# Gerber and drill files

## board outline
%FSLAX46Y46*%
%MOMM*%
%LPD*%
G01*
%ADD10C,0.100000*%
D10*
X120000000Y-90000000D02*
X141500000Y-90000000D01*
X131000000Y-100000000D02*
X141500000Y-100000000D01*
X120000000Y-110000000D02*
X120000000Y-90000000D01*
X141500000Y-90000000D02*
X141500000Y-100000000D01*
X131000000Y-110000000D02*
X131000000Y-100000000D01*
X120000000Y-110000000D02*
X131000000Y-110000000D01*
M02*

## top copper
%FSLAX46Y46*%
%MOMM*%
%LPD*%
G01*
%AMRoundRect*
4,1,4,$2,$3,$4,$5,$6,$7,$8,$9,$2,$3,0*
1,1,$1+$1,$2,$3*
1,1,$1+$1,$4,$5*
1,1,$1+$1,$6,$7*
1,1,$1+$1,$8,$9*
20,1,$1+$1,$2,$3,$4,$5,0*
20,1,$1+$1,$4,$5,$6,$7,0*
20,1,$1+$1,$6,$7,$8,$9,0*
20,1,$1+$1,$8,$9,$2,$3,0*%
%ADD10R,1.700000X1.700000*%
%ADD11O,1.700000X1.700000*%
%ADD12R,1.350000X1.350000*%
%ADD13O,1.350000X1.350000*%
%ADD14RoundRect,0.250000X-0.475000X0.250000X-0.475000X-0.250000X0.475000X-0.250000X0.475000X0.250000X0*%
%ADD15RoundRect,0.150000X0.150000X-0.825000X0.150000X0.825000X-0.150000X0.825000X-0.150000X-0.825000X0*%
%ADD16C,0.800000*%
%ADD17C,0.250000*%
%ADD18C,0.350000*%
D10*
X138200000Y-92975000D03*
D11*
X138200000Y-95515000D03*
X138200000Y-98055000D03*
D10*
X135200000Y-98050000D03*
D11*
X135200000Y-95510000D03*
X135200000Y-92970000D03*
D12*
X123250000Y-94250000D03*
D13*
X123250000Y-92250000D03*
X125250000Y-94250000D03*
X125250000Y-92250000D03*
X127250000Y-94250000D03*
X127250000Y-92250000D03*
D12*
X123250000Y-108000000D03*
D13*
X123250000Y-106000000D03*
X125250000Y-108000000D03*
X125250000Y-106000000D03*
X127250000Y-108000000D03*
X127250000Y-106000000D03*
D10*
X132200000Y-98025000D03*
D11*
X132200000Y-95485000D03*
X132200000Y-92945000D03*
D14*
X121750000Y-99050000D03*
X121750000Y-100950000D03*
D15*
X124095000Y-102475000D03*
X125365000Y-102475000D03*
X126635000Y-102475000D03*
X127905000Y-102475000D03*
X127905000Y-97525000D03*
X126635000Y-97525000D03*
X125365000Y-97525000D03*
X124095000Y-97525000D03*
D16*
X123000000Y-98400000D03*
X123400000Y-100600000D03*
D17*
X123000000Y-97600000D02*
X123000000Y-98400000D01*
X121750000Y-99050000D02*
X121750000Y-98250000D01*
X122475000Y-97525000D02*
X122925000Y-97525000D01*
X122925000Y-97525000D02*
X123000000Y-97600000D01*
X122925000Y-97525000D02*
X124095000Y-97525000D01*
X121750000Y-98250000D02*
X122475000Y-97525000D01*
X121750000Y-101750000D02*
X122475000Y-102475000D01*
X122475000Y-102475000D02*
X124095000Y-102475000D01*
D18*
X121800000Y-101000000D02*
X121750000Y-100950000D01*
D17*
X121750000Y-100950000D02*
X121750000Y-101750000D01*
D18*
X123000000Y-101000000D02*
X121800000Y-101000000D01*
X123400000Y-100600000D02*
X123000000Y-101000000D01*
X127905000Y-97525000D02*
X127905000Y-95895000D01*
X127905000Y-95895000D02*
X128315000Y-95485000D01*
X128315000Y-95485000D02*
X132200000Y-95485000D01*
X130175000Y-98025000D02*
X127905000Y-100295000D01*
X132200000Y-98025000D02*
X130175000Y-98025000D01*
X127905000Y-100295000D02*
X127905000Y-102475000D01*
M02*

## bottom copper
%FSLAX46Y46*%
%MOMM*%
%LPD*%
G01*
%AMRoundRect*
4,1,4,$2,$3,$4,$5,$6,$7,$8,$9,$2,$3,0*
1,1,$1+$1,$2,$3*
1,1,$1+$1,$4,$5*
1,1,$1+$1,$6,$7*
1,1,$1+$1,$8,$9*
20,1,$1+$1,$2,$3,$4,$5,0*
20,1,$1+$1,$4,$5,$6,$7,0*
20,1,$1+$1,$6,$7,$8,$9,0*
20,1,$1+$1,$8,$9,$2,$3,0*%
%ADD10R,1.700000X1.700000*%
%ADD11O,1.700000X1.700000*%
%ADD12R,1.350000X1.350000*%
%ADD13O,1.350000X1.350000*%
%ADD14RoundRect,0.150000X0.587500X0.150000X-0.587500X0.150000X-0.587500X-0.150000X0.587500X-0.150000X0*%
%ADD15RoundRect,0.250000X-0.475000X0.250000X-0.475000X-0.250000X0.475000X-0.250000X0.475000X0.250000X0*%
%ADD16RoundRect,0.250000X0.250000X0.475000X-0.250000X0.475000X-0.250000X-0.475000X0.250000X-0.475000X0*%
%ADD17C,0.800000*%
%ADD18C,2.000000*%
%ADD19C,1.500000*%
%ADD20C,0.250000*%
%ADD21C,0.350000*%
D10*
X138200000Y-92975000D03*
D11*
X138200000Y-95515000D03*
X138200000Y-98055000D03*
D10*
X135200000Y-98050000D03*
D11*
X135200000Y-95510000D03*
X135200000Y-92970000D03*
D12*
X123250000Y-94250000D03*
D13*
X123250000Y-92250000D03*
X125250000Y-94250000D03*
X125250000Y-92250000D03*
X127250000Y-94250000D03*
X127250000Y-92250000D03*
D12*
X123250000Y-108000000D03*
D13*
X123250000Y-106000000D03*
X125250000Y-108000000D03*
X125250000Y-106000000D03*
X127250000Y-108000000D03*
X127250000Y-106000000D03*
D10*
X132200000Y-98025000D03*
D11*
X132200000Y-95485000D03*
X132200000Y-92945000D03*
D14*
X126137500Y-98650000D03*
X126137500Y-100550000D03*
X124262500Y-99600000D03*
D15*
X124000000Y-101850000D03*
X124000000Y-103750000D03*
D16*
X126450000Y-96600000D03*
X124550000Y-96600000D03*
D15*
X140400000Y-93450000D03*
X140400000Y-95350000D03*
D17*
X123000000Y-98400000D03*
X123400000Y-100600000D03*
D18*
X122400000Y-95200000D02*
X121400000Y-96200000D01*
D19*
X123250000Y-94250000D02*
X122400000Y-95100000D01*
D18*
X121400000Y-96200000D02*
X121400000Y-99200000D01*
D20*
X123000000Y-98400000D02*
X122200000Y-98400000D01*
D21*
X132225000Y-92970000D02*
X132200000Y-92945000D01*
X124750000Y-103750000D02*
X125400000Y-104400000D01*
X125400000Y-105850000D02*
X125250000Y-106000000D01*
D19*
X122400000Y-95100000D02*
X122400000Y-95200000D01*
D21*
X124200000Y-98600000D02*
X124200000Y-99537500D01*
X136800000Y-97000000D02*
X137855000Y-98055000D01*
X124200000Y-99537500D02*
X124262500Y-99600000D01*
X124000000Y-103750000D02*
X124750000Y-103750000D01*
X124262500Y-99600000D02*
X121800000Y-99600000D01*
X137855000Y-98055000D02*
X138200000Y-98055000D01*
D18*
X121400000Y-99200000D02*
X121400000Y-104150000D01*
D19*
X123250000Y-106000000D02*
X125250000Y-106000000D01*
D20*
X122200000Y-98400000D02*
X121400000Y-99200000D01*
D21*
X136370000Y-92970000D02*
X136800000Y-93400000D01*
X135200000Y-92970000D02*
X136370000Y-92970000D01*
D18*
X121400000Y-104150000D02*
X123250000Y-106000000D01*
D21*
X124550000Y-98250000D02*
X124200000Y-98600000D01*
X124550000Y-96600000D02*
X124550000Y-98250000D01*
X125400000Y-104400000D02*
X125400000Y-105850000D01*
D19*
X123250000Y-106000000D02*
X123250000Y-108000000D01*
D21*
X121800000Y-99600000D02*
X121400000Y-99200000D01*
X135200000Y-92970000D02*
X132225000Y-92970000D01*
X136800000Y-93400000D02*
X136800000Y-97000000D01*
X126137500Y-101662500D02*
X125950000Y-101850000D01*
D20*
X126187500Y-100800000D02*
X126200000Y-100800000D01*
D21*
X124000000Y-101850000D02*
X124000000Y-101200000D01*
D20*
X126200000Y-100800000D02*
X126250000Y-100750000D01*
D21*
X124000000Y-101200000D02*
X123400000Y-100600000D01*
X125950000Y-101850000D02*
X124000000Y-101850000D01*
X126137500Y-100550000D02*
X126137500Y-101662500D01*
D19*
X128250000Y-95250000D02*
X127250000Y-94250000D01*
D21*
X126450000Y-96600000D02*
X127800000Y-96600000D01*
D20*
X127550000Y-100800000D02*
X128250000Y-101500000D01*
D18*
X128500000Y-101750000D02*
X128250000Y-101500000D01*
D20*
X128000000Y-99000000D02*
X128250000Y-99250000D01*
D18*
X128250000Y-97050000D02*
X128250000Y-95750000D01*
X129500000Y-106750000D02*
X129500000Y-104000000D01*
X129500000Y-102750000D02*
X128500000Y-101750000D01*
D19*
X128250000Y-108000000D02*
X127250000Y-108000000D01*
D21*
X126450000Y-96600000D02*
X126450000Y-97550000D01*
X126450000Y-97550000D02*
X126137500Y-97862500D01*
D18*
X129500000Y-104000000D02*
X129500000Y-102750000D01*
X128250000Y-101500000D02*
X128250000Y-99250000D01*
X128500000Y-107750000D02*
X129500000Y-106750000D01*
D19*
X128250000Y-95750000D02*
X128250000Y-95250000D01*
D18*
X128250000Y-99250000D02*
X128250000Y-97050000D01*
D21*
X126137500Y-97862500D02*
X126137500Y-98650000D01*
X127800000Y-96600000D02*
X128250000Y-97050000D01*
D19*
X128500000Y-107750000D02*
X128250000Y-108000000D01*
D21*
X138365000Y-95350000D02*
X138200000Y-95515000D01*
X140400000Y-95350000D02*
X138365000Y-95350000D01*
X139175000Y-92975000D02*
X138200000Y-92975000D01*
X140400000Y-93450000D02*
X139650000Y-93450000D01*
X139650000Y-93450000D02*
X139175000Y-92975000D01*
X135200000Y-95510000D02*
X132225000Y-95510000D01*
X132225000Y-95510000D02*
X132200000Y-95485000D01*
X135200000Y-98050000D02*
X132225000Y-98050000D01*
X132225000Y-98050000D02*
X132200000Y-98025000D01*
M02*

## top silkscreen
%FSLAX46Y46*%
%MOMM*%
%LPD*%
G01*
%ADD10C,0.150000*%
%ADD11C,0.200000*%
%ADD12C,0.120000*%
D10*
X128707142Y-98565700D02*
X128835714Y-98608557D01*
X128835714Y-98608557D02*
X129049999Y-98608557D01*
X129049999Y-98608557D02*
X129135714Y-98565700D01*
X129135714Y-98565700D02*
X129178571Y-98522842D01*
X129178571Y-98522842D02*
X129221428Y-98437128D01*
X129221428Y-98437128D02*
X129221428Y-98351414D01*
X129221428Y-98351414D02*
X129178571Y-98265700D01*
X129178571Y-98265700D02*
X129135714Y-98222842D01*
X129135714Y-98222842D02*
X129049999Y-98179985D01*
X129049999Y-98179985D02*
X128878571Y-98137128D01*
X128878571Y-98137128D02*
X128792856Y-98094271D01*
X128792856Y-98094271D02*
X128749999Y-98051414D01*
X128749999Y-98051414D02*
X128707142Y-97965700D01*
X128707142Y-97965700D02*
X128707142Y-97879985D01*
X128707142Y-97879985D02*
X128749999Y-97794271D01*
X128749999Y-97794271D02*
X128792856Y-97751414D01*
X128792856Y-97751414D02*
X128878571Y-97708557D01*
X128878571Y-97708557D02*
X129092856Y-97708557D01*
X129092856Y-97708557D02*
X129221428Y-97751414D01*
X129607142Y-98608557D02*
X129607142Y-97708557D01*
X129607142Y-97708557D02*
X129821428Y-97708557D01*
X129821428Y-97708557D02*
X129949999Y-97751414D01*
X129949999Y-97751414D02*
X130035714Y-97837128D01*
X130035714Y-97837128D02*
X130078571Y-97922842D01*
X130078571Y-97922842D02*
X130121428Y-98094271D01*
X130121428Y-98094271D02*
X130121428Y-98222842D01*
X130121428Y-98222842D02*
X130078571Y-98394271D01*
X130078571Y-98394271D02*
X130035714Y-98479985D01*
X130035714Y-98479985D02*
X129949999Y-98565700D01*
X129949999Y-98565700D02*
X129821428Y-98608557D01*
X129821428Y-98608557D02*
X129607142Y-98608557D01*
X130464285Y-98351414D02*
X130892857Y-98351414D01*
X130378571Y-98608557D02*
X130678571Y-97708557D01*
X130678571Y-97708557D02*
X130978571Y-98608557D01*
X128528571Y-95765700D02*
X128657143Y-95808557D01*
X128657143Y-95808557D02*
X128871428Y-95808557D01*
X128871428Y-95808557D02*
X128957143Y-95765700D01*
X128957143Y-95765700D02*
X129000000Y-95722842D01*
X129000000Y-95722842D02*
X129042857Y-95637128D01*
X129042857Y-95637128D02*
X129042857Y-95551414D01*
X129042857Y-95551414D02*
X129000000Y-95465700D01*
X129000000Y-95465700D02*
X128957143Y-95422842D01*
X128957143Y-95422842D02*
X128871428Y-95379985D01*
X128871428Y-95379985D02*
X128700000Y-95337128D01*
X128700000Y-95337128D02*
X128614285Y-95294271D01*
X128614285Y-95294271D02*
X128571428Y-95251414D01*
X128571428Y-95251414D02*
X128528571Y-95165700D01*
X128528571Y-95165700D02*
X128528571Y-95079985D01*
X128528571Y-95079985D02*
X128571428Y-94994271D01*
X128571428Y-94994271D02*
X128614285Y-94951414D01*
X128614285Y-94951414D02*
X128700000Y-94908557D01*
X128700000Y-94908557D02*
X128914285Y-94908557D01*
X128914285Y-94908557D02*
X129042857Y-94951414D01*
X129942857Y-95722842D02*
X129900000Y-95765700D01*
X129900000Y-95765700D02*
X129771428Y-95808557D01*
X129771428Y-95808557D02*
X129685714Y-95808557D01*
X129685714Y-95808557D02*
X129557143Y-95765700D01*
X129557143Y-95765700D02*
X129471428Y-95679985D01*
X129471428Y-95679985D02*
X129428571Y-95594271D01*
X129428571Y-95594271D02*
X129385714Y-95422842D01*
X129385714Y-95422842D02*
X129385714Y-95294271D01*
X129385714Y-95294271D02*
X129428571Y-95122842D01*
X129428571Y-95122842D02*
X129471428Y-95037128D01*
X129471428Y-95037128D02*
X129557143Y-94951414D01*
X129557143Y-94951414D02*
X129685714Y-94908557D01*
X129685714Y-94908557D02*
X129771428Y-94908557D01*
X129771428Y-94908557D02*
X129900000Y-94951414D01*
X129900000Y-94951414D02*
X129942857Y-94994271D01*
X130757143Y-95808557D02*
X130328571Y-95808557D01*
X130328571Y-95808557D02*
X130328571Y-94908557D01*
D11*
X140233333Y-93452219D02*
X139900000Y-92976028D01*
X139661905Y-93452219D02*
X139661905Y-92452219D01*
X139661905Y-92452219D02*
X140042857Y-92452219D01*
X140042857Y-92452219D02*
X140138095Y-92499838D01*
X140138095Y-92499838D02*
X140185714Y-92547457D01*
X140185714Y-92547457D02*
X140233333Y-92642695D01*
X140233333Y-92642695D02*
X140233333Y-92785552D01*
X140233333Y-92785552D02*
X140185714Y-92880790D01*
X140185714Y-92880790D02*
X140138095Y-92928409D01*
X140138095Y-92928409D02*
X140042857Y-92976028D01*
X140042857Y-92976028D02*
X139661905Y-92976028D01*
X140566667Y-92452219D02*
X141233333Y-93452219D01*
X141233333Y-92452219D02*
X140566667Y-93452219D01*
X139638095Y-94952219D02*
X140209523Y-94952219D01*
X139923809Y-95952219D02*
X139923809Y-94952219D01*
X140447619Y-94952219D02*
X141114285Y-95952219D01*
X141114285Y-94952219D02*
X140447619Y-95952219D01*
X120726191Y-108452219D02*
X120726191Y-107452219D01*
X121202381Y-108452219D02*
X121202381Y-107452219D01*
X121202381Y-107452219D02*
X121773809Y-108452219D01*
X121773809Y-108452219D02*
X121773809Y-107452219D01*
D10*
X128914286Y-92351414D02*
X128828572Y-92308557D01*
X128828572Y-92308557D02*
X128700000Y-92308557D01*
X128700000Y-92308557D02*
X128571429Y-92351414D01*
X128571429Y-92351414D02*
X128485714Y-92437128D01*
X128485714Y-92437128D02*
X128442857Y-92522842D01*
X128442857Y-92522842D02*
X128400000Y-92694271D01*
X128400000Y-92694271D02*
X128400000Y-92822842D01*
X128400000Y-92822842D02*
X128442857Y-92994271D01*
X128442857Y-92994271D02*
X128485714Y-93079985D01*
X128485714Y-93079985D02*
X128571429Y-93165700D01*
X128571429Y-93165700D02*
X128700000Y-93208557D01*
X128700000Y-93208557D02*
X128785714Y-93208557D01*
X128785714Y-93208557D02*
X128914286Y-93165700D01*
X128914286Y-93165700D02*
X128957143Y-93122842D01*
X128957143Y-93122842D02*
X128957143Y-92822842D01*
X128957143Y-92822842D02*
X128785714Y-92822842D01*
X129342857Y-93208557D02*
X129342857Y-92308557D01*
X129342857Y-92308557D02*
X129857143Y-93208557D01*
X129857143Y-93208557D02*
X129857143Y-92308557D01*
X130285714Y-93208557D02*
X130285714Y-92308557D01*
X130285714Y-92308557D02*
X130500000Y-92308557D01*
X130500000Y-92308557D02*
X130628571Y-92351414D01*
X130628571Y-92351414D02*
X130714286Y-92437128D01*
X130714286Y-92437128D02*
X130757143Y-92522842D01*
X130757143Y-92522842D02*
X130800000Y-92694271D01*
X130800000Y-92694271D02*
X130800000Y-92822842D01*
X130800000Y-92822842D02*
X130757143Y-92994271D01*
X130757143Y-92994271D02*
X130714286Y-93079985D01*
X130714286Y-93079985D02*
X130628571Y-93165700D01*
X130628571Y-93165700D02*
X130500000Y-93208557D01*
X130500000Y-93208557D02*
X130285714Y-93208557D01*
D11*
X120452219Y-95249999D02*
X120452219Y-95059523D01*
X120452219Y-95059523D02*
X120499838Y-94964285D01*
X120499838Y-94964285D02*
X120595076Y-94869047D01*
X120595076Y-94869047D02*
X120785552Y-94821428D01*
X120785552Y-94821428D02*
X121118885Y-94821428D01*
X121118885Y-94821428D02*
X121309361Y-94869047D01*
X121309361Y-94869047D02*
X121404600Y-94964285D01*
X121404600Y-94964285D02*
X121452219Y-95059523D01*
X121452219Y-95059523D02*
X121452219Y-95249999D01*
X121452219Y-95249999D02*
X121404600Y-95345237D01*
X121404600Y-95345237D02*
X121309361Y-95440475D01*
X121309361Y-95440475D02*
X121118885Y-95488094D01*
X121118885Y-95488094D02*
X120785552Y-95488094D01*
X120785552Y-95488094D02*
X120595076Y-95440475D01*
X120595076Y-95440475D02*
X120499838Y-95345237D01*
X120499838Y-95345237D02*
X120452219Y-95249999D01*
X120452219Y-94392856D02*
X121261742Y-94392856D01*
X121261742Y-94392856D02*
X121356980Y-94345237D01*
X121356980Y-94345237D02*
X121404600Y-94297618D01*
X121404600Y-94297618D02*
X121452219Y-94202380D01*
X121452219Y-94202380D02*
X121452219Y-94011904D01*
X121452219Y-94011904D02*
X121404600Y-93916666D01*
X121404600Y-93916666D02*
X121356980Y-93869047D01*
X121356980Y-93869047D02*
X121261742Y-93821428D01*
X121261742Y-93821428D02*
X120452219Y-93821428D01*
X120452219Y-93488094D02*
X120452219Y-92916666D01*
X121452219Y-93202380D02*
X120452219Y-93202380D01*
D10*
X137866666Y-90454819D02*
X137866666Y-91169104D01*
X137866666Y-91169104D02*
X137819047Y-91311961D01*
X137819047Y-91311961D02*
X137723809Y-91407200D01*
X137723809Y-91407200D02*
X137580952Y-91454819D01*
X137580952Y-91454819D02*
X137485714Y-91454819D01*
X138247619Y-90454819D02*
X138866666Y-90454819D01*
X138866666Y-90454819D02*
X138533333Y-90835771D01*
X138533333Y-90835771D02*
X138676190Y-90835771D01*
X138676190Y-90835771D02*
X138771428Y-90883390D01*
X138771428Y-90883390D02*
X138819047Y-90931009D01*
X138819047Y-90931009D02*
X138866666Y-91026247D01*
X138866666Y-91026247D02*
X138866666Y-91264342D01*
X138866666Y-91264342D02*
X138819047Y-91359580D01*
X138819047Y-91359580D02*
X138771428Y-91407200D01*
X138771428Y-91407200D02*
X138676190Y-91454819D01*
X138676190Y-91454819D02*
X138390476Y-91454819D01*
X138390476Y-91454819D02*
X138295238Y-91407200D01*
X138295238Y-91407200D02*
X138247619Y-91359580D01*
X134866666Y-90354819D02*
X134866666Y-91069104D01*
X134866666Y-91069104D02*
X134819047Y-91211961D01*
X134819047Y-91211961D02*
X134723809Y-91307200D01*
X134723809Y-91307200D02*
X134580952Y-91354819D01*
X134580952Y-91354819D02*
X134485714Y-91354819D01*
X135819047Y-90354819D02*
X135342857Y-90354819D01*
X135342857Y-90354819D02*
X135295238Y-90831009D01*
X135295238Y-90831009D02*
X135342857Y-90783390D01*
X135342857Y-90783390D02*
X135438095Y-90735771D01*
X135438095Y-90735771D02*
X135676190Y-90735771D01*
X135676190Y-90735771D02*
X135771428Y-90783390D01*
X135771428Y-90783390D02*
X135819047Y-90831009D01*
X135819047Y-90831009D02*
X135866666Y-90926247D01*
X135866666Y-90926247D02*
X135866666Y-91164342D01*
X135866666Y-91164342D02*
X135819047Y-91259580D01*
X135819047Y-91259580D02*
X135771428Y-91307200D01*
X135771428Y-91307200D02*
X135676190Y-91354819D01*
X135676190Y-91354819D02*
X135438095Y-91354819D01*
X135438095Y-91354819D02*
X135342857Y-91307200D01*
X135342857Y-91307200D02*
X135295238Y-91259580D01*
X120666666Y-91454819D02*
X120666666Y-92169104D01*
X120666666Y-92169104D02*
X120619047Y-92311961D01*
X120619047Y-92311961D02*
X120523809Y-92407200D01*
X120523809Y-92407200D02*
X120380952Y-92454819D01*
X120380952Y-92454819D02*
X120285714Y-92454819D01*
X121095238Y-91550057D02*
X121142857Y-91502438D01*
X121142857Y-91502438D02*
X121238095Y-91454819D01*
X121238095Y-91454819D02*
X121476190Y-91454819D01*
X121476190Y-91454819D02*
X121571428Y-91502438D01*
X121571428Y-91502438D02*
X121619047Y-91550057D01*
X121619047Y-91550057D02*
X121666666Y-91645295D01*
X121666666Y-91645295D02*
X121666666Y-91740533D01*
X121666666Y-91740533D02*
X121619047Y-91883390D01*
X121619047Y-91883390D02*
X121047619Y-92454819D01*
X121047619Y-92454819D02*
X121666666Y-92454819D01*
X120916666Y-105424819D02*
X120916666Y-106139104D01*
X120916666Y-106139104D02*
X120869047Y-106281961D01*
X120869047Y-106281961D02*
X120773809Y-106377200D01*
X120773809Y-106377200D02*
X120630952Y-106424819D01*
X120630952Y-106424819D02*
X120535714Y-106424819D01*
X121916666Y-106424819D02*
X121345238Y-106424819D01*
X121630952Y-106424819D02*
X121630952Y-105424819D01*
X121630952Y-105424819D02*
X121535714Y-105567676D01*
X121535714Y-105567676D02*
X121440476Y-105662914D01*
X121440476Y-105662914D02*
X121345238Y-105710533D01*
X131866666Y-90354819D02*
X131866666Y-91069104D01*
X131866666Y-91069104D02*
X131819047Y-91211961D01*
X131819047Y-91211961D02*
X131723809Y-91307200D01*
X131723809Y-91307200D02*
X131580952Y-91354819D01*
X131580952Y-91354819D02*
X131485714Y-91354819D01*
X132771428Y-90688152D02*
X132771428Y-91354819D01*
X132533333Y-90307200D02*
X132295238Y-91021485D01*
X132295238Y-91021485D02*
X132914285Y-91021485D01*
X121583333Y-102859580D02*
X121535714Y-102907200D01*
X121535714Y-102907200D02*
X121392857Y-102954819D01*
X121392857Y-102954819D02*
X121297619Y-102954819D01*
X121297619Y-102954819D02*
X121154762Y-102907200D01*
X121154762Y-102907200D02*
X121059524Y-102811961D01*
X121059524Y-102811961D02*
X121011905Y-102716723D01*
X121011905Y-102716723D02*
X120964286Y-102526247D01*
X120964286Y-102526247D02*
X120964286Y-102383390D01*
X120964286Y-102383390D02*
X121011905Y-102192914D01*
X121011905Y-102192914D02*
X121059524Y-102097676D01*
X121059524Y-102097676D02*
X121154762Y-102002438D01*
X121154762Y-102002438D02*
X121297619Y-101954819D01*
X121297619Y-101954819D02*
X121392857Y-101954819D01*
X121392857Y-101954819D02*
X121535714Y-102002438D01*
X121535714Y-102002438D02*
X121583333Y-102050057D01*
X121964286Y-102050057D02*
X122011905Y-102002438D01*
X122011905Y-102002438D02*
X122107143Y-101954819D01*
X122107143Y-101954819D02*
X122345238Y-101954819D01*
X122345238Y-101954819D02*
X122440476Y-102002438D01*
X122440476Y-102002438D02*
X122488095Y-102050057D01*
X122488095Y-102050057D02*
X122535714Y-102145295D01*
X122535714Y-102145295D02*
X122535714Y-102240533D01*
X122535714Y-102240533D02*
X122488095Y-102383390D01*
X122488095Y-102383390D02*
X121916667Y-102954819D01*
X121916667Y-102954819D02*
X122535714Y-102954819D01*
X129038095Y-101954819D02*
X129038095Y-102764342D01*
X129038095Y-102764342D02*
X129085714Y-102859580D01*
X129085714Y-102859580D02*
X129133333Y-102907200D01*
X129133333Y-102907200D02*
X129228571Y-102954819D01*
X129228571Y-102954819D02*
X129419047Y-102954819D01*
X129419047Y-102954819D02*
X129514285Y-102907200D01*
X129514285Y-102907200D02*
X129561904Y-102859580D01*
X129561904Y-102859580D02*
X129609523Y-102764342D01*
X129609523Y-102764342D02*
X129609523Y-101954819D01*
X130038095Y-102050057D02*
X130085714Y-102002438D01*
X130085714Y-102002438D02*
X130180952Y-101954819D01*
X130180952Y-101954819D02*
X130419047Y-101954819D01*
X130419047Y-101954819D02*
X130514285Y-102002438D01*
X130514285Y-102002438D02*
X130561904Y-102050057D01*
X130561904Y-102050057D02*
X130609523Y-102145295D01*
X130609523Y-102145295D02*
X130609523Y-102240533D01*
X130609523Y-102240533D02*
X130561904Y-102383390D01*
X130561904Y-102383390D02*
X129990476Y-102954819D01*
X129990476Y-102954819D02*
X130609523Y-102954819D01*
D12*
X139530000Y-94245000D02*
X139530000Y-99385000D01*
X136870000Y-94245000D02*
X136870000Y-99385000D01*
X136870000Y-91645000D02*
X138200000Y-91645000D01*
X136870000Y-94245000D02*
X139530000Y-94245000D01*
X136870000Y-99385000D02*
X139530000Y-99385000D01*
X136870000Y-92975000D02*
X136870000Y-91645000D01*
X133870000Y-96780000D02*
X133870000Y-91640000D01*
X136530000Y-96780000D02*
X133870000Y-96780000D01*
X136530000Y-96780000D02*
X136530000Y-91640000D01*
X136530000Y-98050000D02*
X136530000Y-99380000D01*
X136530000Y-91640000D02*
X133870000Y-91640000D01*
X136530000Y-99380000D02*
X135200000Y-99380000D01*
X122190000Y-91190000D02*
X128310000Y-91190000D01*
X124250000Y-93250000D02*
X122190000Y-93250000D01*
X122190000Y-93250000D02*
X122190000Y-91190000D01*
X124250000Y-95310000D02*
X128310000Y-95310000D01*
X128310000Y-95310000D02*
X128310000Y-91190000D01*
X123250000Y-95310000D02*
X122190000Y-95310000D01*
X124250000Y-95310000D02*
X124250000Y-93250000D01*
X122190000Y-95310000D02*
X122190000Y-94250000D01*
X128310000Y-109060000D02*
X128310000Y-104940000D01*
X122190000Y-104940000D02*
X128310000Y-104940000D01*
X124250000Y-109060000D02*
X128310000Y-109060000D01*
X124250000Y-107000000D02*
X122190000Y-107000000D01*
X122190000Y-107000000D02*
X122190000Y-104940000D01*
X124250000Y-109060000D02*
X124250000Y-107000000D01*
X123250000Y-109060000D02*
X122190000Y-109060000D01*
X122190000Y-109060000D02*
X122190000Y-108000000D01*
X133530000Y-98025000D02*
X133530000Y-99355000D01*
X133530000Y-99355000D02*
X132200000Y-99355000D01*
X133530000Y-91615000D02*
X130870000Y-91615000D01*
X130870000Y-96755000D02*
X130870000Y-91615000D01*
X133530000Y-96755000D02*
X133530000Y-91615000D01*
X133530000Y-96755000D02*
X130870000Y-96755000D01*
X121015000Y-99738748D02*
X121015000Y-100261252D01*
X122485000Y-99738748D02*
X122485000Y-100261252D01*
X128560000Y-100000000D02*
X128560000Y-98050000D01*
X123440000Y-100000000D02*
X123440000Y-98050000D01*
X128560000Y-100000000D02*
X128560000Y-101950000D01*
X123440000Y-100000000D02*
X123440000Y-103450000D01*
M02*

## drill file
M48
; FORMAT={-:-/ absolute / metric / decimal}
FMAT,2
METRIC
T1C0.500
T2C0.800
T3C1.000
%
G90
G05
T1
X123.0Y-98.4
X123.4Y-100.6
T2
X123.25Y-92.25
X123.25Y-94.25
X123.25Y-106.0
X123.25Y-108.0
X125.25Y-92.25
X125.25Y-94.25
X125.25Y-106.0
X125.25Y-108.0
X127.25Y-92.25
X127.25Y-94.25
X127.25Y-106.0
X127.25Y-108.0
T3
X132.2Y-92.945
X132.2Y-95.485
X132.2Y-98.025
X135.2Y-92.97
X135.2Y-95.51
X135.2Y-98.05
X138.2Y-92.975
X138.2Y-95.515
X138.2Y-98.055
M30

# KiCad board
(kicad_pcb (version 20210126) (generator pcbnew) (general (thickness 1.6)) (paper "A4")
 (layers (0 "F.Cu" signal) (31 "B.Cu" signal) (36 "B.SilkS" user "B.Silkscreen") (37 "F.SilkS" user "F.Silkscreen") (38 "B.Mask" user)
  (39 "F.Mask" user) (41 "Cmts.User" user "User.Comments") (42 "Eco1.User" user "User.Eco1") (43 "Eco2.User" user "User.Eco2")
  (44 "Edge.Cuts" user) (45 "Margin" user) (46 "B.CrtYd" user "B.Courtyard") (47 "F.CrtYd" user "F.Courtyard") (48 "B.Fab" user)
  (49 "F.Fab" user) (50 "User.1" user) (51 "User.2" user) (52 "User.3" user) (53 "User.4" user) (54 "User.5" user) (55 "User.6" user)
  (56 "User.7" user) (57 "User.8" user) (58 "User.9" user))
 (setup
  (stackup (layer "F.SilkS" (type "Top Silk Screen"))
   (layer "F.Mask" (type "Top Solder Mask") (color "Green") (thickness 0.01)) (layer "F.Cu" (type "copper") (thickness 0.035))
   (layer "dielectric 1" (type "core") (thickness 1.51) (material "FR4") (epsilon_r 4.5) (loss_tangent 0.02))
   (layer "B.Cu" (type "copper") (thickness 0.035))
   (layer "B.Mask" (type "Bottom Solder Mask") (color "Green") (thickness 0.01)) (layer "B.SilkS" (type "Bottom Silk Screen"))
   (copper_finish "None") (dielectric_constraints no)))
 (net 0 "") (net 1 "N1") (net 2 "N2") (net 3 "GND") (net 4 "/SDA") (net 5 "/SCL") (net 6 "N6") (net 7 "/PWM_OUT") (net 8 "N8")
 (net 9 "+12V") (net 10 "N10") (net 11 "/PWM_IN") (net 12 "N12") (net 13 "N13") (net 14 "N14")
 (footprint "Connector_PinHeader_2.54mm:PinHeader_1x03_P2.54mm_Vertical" (layer "F.Cu") (at 138.2 92.975)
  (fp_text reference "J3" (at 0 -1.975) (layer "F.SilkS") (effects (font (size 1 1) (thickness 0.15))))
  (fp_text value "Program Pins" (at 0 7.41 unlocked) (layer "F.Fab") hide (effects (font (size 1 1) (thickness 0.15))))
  (fp_line (start 1.33 1.27) (end 1.33 6.41) (layer "F.SilkS") (width 0.12))
  (fp_line (start -1.33 1.27) (end -1.33 6.41) (layer "F.SilkS") (width 0.12))
  (fp_line (start -1.33 -1.33) (end 0 -1.33) (layer "F.SilkS") (width 0.12))
  (fp_line (start -1.33 1.27) (end 1.33 1.27) (layer "F.SilkS") (width 0.12))
  (fp_line (start -1.33 6.41) (end 1.33 6.41) (layer "F.SilkS") (width 0.12))
  (fp_line (start -1.33 0) (end -1.33 -1.33) (layer "F.SilkS") (width 0.12))
  (pad "1" thru_hole rect (at 0 0) (locked) (size 1.7 1.7) (drill 1) (layers *.Cu *.Mask) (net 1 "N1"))
  (pad "2" thru_hole oval (at 0 2.54) (locked) (size 1.7 1.7) (drill 1) (layers *.Cu *.Mask) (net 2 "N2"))
  (pad "3" thru_hole oval (at 0 5.08) (locked) (size 1.7 1.7) (drill 1) (layers *.Cu *.Mask) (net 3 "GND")))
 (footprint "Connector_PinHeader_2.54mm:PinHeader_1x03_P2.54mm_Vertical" (layer "F.Cu") (at 135.2 98.05 180)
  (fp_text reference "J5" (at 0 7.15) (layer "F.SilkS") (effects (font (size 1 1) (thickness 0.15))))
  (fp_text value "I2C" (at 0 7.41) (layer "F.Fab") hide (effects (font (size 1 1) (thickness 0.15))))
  (fp_line (start 1.33 1.27) (end 1.33 6.41) (layer "F.SilkS") (width 0.12))
  (fp_line (start -1.33 1.27) (end 1.33 1.27) (layer "F.SilkS") (width 0.12))
  (fp_line (start -1.33 1.27) (end -1.33 6.41) (layer "F.SilkS") (width 0.12))
  (fp_line (start -1.33 0) (end -1.33 -1.33) (layer "F.SilkS") (width 0.12))
  (fp_line (start -1.33 6.41) (end 1.33 6.41) (layer "F.SilkS") (width 0.12))
  (fp_line (start -1.33 -1.33) (end 0 -1.33) (layer "F.SilkS") (width 0.12))
  (pad "1" thru_hole rect (at 0 0 180) (locked) (size 1.7 1.7) (drill 1) (layers *.Cu *.Mask) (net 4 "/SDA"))
  (pad "2" thru_hole oval (at 0 2.54 180) (locked) (size 1.7 1.7) (drill 1) (layers *.Cu *.Mask) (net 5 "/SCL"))
  (pad "3" thru_hole oval (at 0 5.08 180) (locked) (size 1.7 1.7) (drill 1) (layers *.Cu *.Mask) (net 3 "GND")))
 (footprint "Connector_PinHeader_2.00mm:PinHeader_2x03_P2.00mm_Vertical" (layer "F.Cu") (at 123.25 94.25 90)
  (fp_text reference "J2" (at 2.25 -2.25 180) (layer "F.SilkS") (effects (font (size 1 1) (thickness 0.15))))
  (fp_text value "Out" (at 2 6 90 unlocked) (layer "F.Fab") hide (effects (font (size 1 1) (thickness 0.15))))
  (fp_line (start 3.06 -1.06) (end 3.06 5.06) (layer "F.SilkS") (width 0.12))
  (fp_line (start 1 1) (end 1 -1.06) (layer "F.SilkS") (width 0.12))
  (fp_line (start 1 -1.06) (end 3.06 -1.06) (layer "F.SilkS") (width 0.12))
  (fp_line (start -1.06 1) (end -1.06 5.06) (layer "F.SilkS") (width 0.12))
  (fp_line (start -1.06 5.06) (end 3.06 5.06) (layer "F.SilkS") (width 0.12))
  (fp_line (start -1.06 0) (end -1.06 -1.06) (layer "F.SilkS") (width 0.12))
  (fp_line (start -1.06 1) (end 1 1) (layer "F.SilkS") (width 0.12))
  (fp_line (start -1.06 -1.06) (end 0 -1.06) (layer "F.SilkS") (width 0.12))
  (pad "1" thru_hole rect (at 0 0 90) (locked) (size 1.35 1.35) (drill 0.8) (layers *.Cu *.Mask) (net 3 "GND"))
  (pad "2" thru_hole oval (at 2 0 90) (locked) (size 1.35 1.35) (drill 0.8) (layers *.Cu *.Mask) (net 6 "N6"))
  (pad "3" thru_hole oval (at 0 2 90) (locked) (size 1.35 1.35) (drill 0.8) (layers *.Cu *.Mask) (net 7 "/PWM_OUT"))
  (pad "4" thru_hole oval (at 2 2 90) (locked) (size 1.35 1.35) (drill 0.8) (layers *.Cu *.Mask) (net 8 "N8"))
  (pad "5" thru_hole oval (at 0 4 90) (locked) (size 1.35 1.35) (drill 0.8) (layers *.Cu *.Mask) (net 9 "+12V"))
  (pad "6" thru_hole oval (at 2 4 90) (locked) (size 1.35 1.35) (drill 0.8) (layers *.Cu *.Mask) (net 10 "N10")))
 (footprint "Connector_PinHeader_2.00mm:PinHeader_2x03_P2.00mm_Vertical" (layer "F.Cu") (at 123.25 108 90)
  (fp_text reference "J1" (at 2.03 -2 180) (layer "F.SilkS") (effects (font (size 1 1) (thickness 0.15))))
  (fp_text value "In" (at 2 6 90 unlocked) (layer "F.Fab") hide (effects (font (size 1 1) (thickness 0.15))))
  (fp_line (start -1.06 5.06) (end 3.06 5.06) (layer "F.SilkS") (width 0.12))
  (fp_line (start 3.06 -1.06) (end 3.06 5.06) (layer "F.SilkS") (width 0.12))
  (fp_line (start -1.06 1) (end -1.06 5.06) (layer "F.SilkS") (width 0.12))
  (fp_line (start 1 1) (end 1 -1.06) (layer "F.SilkS") (width 0.12))
  (fp_line (start 1 -1.06) (end 3.06 -1.06) (layer "F.SilkS") (width 0.12))
  (fp_line (start -1.06 1) (end 1 1) (layer "F.SilkS") (width 0.12))
  (fp_line (start -1.06 0) (end -1.06 -1.06) (layer "F.SilkS") (width 0.12))
  (fp_line (start -1.06 -1.06) (end 0 -1.06) (layer "F.SilkS") (width 0.12))
  (pad "1" thru_hole rect (at 0 0 90) (locked) (size 1.35 1.35) (drill 0.8) (layers *.Cu *.Mask) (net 3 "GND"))
  (pad "2" thru_hole oval (at 2 0 90) (locked) (size 1.35 1.35) (drill 0.8) (layers *.Cu *.Mask) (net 3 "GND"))
  (pad "3" thru_hole oval (at 0 2 90) (locked) (size 1.35 1.35) (drill 0.8) (layers *.Cu *.Mask) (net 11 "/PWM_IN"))
  (pad "4" thru_hole oval (at 2 2 90) (locked) (size 1.35 1.35) (drill 0.8) (layers *.Cu *.Mask) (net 3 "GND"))
  (pad "5" thru_hole oval (at 0 4 90) (locked) (size 1.35 1.35) (drill 0.8) (layers *.Cu *.Mask) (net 9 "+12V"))
  (pad "6" thru_hole oval (at 2 4 90) (locked) (size 1.35 1.35) (drill 0.8) (layers *.Cu *.Mask) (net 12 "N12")))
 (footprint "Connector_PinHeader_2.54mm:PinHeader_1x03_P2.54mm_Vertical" (layer "F.Cu") (at 132.2 98.025 180)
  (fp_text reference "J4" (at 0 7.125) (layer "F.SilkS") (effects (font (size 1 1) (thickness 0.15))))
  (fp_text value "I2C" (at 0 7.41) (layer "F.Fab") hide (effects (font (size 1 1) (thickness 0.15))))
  (fp_line (start -1.33 0) (end -1.33 -1.33) (layer "F.SilkS") (width 0.12))
  (fp_line (start -1.33 -1.33) (end 0 -1.33) (layer "F.SilkS") (width 0.12))
  (fp_line (start -1.33 6.41) (end 1.33 6.41) (layer "F.SilkS") (width 0.12))
  (fp_line (start 1.33 1.27) (end 1.33 6.41) (layer "F.SilkS") (width 0.12))
  (fp_line (start -1.33 1.27) (end -1.33 6.41) (layer "F.SilkS") (width 0.12))
  (fp_line (start -1.33 1.27) (end 1.33 1.27) (layer "F.SilkS") (width 0.12))
  (pad "1" thru_hole rect (at 0 0 180) (locked) (size 1.7 1.7) (drill 1) (layers *.Cu *.Mask) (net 4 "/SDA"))
  (pad "2" thru_hole oval (at 0 2.54 180) (locked) (size 1.7 1.7) (drill 1) (layers *.Cu *.Mask) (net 5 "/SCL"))
  (pad "3" thru_hole oval (at 0 5.08 180) (locked) (size 1.7 1.7) (drill 1) (layers *.Cu *.Mask) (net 3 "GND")))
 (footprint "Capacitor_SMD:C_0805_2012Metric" (layer "F.Cu") (at 121.75 100 -90)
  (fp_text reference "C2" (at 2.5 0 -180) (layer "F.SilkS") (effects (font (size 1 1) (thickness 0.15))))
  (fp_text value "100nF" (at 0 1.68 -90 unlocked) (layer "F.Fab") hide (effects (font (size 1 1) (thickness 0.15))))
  (fp_line (start -0.261252 0.735) (end 0.261252 0.735) (layer "F.SilkS") (width 0.12))
  (fp_line (start -0.261252 -0.735) (end 0.261252 -0.735) (layer "F.SilkS") (width 0.12))
  (pad "1" smd roundrect (at -0.95 0 270) (locked) (size 1 1.45) (layers "F.Cu" "F.Paste" "F.Mask") (roundrect_rratio 0.25) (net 3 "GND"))
  (pad "2" smd roundrect (at 0.95 0 270) (locked) (size 1 1.45) (layers "F.Cu" "F.Paste" "F.Mask") (roundrect_rratio 0.25) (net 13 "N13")))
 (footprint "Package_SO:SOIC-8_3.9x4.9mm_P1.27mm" (layer "F.Cu") (at 126 100 90)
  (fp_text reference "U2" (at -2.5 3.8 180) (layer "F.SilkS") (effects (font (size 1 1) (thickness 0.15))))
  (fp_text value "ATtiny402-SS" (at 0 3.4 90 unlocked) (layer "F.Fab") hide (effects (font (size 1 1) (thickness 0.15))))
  (fp_line (start 0 2.56) (end 1.95 2.56) (layer "F.SilkS") (width 0.12))
  (fp_line (start 0 -2.56) (end 1.95 -2.56) (layer "F.SilkS") (width 0.12))
  (fp_line (start 0 2.56) (end -1.95 2.56) (layer "F.SilkS") (width 0.12))
  (fp_line (start 0 -2.56) (end -3.45 -2.56) (layer "F.SilkS") (width 0.12))
  (pad "1" smd roundrect (at -2.475 -1.905 90) (locked) (size 1.95 0.6) (layers "F.Cu" "F.Paste" "F.Mask") (roundrect_rratio 0.25)
   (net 13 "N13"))
  (pad "2" smd roundrect (at -2.475 -0.635 90) (locked) (size 1.95 0.6) (layers "F.Cu" "F.Paste" "F.Mask") (roundrect_rratio 0.25)
   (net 11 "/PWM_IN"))
  (pad "3" smd roundrect (at -2.475 0.635 90) (locked) (size 1.95 0.6) (layers "F.Cu" "F.Paste" "F.Mask") (roundrect_rratio 0.25)
   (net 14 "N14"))
  (pad "4" smd roundrect (at -2.475 1.905 90) (locked) (size 1.95 0.6) (layers "F.Cu" "F.Paste" "F.Mask") (roundrect_rratio 0.25)
   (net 4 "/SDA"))
  (pad "5" smd roundrect (at 2.475 1.905 90) (locked) (size 1.95 0.6) (layers "F.Cu" "F.Paste" "F.Mask") (roundrect_rratio 0.25)
   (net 5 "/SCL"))
  (pad "6" smd roundrect (at 2.475 0.635 90) (locked) (size 1.95 0.6) (layers "F.Cu" "F.Paste" "F.Mask") (roundrect_rratio 0.25)
   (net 2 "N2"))
  (pad "7" smd roundrect (at 2.475 -0.635 90) (locked) (size 1.95 0.6) (layers "F.Cu" "F.Paste" "F.Mask") (roundrect_rratio 0.25)
   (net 7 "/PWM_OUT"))
  (pad "8" smd roundrect (at 2.475 -1.905 90) (locked) (size 1.95 0.6) (layers "F.Cu" "F.Paste" "F.Mask") (roundrect_rratio 0.25)
   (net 3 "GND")))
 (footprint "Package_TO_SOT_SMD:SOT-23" (layer "B.Cu") (at 125.2 99.6 180)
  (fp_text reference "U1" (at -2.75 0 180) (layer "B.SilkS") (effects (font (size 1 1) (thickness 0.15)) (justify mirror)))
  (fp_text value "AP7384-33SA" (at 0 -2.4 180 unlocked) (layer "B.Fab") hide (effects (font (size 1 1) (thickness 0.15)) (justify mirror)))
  (pad "1" smd roundrect (at -0.9375 0.95 180) (locked) (size 1.475 0.6) (layers "B.Cu" "B.Paste" "B.Mask") (roundrect_rratio 0.25)
   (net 9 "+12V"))
  (pad "2" smd roundrect (at -0.9375 -0.95 180) (locked) (size 1.475 0.6) (layers "B.Cu" "B.Paste" "B.Mask") (roundrect_rratio 0.25)
   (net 13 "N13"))
  (pad "3" smd roundrect (at 0.9375 0 180) (locked) (size 1.475 0.6) (layers "B.Cu" "B.Paste" "B.Mask") (roundrect_rratio 0.25)
   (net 3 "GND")))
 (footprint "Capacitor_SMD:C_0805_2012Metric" (layer "B.Cu") (at 124 102.8 -90)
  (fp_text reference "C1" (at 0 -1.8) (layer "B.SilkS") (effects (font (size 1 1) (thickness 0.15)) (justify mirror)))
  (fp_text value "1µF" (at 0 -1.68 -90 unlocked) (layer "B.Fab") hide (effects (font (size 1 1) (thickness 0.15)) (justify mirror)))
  (pad "1" smd roundrect (at -0.95 0 270) (locked) (size 1 1.45) (layers "B.Cu" "B.Paste" "B.Mask") (roundrect_rratio 0.25) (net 13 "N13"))
  (pad "2" smd roundrect (at 0.95 0 270) (locked) (size 1 1.45) (layers "B.Cu" "B.Paste" "B.Mask") (roundrect_rratio 0.25) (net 3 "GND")))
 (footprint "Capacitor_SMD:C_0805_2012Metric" (layer "B.Cu") (at 125.5 96.6 180)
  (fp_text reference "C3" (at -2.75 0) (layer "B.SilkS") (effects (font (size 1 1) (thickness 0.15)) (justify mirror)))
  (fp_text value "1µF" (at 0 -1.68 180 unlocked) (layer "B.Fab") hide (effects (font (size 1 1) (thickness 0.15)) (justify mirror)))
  (pad "1" smd roundrect (at -0.95 0 180) (locked) (size 1 1.45) (layers "B.Cu" "B.Paste" "B.Mask") (roundrect_rratio 0.25) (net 9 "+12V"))
  (pad "2" smd roundrect (at 0.95 0 180) (locked) (size 1 1.45) (layers "B.Cu" "B.Paste" "B.Mask") (roundrect_rratio 0.25) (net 3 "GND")))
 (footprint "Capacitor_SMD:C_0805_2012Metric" (layer "B.Cu") (at 140.4 94.4 -90)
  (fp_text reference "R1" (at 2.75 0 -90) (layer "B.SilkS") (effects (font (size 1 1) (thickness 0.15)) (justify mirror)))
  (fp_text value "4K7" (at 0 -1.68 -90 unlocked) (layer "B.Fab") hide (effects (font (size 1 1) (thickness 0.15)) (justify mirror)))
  (pad "1" smd roundrect (at -0.95 0 270) (locked) (size 1 1.45) (layers "B.Cu" "B.Paste" "B.Mask") (roundrect_rratio 0.25) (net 1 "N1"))
  (pad "2" smd roundrect (at 0.95 0 270) (locked) (size 1 1.45) (layers "B.Cu" "B.Paste" "B.Mask") (roundrect_rratio 0.25) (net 2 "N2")))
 (gr_line (start 120 90) (end 141.5 90) (layer "Edge.Cuts") (width 0.1))
 (gr_line (start 131 100) (end 141.5 100) (layer "Edge.Cuts") (width 0.1))
 (gr_line (start 120 110) (end 120 90) (layer "Edge.Cuts") (width 0.1))
 (gr_line (start 141.5 90) (end 141.5 100) (layer "Edge.Cuts") (width 0.1))
 (gr_line (start 131 110) (end 131 100) (layer "Edge.Cuts") (width 0.1))
 (gr_line (start 120 110) (end 131 110) (layer "Edge.Cuts") (width 0.1))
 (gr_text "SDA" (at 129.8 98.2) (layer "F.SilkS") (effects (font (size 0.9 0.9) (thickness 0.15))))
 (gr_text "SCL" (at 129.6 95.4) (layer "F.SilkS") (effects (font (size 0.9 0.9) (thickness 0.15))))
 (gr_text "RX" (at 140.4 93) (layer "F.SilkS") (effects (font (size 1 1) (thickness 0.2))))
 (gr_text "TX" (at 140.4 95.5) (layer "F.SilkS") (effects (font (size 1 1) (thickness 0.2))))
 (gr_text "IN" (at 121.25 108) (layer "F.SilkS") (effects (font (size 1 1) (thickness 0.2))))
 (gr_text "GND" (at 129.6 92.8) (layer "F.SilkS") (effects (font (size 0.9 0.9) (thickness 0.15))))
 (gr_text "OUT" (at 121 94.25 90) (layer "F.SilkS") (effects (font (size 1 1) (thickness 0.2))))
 (segment (start 123 97.6) (end 123 98.4) (width 0.25) (layer "F.Cu") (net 3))
 (segment (start 121.75 99.05) (end 121.75 98.25) (width 0.25) (layer "F.Cu") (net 3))
 (segment (start 122.475 97.525) (end 122.925 97.525) (width 0.25) (layer "F.Cu") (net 3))
 (segment (start 122.925 97.525) (end 123 97.6) (width 0.25) (layer "F.Cu") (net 3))
 (segment (start 122.925 97.525) (end 124.095 97.525) (width 0.25) (layer "F.Cu") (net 3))
 (segment (start 121.75 98.25) (end 122.475 97.525) (width 0.25) (layer "F.Cu") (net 3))
 (via (at 123 98.4) (size 0.8) (drill 0.5) (layers "F.Cu" "B.Cu") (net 3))
 (segment (start 122.4 95.2) (end 121.4 96.2) (width 2) (layer "B.Cu") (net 3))
 (segment (start 123.25 94.25) (end 122.4 95.1) (width 1.5) (layer "B.Cu") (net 3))
 (segment (start 121.4 96.2) (end 121.4 99.2) (width 2) (layer "B.Cu") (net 3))
 (segment (start 123 98.4) (end 122.2 98.4) (width 0.25) (layer "B.Cu") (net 3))
 (segment (start 132.225 92.97) (end 132.2 92.945) (width 0.35) (layer "B.Cu") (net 3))
 (segment (start 124.75 103.75) (end 125.4 104.4) (width 0.35) (layer "B.Cu") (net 3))
 (segment (start 125.4 105.85) (end 125.25 106) (width 0.35) (layer "B.Cu") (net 3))
 (segment (start 122.4 95.1) (end 122.4 95.2) (width 1.5) (layer "B.Cu") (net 3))
 (segment (start 124.2 98.6) (end 124.2 99.5375) (width 0.35) (layer "B.Cu") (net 3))
 (segment (start 136.8 97) (end 137.855 98.055) (width 0.35) (layer "B.Cu") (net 3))
 (segment (start 124.2 99.5375) (end 124.2625 99.6) (width 0.35) (layer "B.Cu") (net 3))
 (segment (start 124 103.75) (end 124.75 103.75) (width 0.35) (layer "B.Cu") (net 3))
 (segment (start 124.2625 99.6) (end 121.8 99.6) (width 0.35) (layer "B.Cu") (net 3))
 (segment (start 137.855 98.055) (end 138.2 98.055) (width 0.35) (layer "B.Cu") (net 3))
 (segment (start 121.4 99.2) (end 121.4 104.15) (width 2) (layer "B.Cu") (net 3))
 (segment (start 123.25 106) (end 125.25 106) (width 1.5) (layer "B.Cu") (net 3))
 (segment (start 122.2 98.4) (end 121.4 99.2) (width 0.25) (layer "B.Cu") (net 3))
 (segment (start 136.37 92.97) (end 136.8 93.4) (width 0.35) (layer "B.Cu") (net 3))
 (segment (start 135.2 92.97) (end 136.37 92.97) (width 0.35) (layer "B.Cu") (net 3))
 (segment (start 121.4 104.15) (end 123.25 106) (width 2) (layer "B.Cu") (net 3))
 (segment (start 124.55 98.25) (end 124.2 98.6) (width 0.35) (layer "B.Cu") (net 3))
 (segment (start 124.55 96.6) (end 124.55 98.25) (width 0.35) (layer "B.Cu") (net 3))
 (segment (start 125.4 104.4) (end 125.4 105.85) (width 0.35) (layer "B.Cu") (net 3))
 (segment (start 123.25 106) (end 123.25 108) (width 1.5) (layer "B.Cu") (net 3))
 (segment (start 121.8 99.6) (end 121.4 99.2) (width 0.35) (layer "B.Cu") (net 3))
 (segment (start 135.2 92.97) (end 132.225 92.97) (width 0.35) (layer "B.Cu") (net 3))
 (segment (start 136.8 93.4) (end 136.8 97) (width 0.35) (layer "B.Cu") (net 3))
 (segment (start 121.75 101.75) (end 122.475 102.475) (width 0.25) (layer "F.Cu") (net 13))
 (segment (start 122.475 102.475) (end 124.095 102.475) (width 0.25) (layer "F.Cu") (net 13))
 (segment (start 121.8 101) (end 121.75 100.95) (width 0.35) (layer "F.Cu") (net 13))
 (segment (start 121.75 100.95) (end 121.75 101.75) (width 0.25) (layer "F.Cu") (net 13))
 (segment (start 123 101) (end 121.8 101) (width 0.35) (layer "F.Cu") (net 13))
 (segment (start 123.4 100.6) (end 123 101) (width 0.35) (layer "F.Cu") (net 13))
 (via (at 123.4 100.6) (size 0.8) (drill 0.5) (layers "F.Cu" "B.Cu") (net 13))
 (segment (start 126.1375 101.6625) (end 125.95 101.85) (width 0.35) (layer "B.Cu") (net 13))
 (segment (start 126.1875 100.8) (end 126.2 100.8) (width 0.25) (layer "B.Cu") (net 13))
 (segment (start 124 101.85) (end 124 101.2) (width 0.35) (layer "B.Cu") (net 13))
 (segment (start 126.2 100.8) (end 126.25 100.75) (width 0.25) (layer "B.Cu") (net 13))
 (segment (start 124 101.2) (end 123.4 100.6) (width 0.35) (layer "B.Cu") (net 13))
 (segment (start 125.95 101.85) (end 124 101.85) (width 0.35) (layer "B.Cu") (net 13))
 (segment (start 126.1375 100.55) (end 126.1375 101.6625) (width 0.35) (layer "B.Cu") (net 13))
 (segment (start 128.25 95.25) (end 127.25 94.25) (width 1.5) (layer "B.Cu") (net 9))
 (segment (start 126.45 96.6) (end 127.8 96.6) (width 0.35) (layer "B.Cu") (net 9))
 (segment (start 127.55 100.8) (end 128.25 101.5) (width 0.25) (layer "B.Cu") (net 9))
 (segment (start 128.5 101.75) (end 128.25 101.5) (width 2) (layer "B.Cu") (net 9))
 (segment (start 128 99) (end 128.25 99.25) (width 0.25) (layer "B.Cu") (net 9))
 (segment (start 128.25 97.05) (end 128.25 95.75) (width 2) (layer "B.Cu") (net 9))
 (segment (start 129.5 106.75) (end 129.5 104) (width 2) (layer "B.Cu") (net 9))
 (segment (start 129.5 102.75) (end 128.5 101.75) (width 2) (layer "B.Cu") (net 9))
 (segment (start 128.25 108) (end 127.25 108) (width 1.5) (layer "B.Cu") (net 9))
 (segment (start 126.45 96.6) (end 126.45 97.55) (width 0.35) (layer "B.Cu") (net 9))
 (segment (start 126.45 97.55) (end 126.1375 97.8625) (width 0.35) (layer "B.Cu") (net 9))
 (segment (start 129.5 104) (end 129.5 102.75) (width 2) (layer "B.Cu") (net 9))
 (segment (start 128.25 101.5) (end 128.25 99.25) (width 2) (layer "B.Cu") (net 9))
 (segment (start 128.5 107.75) (end 129.5 106.75) (width 2) (layer "B.Cu") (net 9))
 (segment (start 128.25 95.75) (end 128.25 95.25) (width 1.5) (layer "B.Cu") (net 9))
 (segment (start 128.25 99.25) (end 128.25 97.05) (width 2) (layer "B.Cu") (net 9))
 (segment (start 126.1375 97.8625) (end 126.1375 98.65) (width 0.35) (layer "B.Cu") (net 9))
 (segment (start 127.8 96.6) (end 128.25 97.05) (width 0.35) (layer "B.Cu") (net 9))
 (segment (start 128.5 107.75) (end 128.25 108) (width 1.5) (layer "B.Cu") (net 9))
 (segment (start 138.365 95.35) (end 138.2 95.515) (width 0.35) (layer "B.Cu") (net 2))
 (segment (start 140.4 95.35) (end 138.365 95.35) (width 0.35) (layer "B.Cu") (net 2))
 (segment (start 139.175 92.975) (end 138.2 92.975) (width 0.35) (layer "B.Cu") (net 1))
 (segment (start 140.4 93.45) (end 139.65 93.45) (width 0.35) (layer "B.Cu") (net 1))
 (segment (start 139.65 93.45) (end 139.175 92.975) (width 0.35) (layer "B.Cu") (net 1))
 (segment (start 127.905 97.525) (end 127.905 95.895) (width 0.35) (layer "F.Cu") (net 5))
 (segment (start 127.905 95.895) (end 128.315 95.485) (width 0.35) (layer "F.Cu") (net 5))
 (segment (start 128.315 95.485) (end 132.2 95.485) (width 0.35) (layer "F.Cu") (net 5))
 (segment (start 135.2 95.51) (end 132.225 95.51) (width 0.35) (layer "B.Cu") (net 5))
 (segment (start 132.225 95.51) (end 132.2 95.485) (width 0.35) (layer "B.Cu") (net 5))
 (segment (start 130.175 98.025) (end 127.905 100.295) (width 0.35) (layer "F.Cu") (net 4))
 (segment (start 132.2 98.025) (end 130.175 98.025) (width 0.35) (layer "F.Cu") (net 4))
 (segment (start 127.905 100.295) (end 127.905 102.475) (width 0.35) (layer "F.Cu") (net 4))
 (segment (start 135.2 98.05) (end 132.225 98.05) (width 0.35) (layer "B.Cu") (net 4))
 (segment (start 132.225 98.05) (end 132.2 98.025) (width 0.35) (layer "B.Cu") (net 4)))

